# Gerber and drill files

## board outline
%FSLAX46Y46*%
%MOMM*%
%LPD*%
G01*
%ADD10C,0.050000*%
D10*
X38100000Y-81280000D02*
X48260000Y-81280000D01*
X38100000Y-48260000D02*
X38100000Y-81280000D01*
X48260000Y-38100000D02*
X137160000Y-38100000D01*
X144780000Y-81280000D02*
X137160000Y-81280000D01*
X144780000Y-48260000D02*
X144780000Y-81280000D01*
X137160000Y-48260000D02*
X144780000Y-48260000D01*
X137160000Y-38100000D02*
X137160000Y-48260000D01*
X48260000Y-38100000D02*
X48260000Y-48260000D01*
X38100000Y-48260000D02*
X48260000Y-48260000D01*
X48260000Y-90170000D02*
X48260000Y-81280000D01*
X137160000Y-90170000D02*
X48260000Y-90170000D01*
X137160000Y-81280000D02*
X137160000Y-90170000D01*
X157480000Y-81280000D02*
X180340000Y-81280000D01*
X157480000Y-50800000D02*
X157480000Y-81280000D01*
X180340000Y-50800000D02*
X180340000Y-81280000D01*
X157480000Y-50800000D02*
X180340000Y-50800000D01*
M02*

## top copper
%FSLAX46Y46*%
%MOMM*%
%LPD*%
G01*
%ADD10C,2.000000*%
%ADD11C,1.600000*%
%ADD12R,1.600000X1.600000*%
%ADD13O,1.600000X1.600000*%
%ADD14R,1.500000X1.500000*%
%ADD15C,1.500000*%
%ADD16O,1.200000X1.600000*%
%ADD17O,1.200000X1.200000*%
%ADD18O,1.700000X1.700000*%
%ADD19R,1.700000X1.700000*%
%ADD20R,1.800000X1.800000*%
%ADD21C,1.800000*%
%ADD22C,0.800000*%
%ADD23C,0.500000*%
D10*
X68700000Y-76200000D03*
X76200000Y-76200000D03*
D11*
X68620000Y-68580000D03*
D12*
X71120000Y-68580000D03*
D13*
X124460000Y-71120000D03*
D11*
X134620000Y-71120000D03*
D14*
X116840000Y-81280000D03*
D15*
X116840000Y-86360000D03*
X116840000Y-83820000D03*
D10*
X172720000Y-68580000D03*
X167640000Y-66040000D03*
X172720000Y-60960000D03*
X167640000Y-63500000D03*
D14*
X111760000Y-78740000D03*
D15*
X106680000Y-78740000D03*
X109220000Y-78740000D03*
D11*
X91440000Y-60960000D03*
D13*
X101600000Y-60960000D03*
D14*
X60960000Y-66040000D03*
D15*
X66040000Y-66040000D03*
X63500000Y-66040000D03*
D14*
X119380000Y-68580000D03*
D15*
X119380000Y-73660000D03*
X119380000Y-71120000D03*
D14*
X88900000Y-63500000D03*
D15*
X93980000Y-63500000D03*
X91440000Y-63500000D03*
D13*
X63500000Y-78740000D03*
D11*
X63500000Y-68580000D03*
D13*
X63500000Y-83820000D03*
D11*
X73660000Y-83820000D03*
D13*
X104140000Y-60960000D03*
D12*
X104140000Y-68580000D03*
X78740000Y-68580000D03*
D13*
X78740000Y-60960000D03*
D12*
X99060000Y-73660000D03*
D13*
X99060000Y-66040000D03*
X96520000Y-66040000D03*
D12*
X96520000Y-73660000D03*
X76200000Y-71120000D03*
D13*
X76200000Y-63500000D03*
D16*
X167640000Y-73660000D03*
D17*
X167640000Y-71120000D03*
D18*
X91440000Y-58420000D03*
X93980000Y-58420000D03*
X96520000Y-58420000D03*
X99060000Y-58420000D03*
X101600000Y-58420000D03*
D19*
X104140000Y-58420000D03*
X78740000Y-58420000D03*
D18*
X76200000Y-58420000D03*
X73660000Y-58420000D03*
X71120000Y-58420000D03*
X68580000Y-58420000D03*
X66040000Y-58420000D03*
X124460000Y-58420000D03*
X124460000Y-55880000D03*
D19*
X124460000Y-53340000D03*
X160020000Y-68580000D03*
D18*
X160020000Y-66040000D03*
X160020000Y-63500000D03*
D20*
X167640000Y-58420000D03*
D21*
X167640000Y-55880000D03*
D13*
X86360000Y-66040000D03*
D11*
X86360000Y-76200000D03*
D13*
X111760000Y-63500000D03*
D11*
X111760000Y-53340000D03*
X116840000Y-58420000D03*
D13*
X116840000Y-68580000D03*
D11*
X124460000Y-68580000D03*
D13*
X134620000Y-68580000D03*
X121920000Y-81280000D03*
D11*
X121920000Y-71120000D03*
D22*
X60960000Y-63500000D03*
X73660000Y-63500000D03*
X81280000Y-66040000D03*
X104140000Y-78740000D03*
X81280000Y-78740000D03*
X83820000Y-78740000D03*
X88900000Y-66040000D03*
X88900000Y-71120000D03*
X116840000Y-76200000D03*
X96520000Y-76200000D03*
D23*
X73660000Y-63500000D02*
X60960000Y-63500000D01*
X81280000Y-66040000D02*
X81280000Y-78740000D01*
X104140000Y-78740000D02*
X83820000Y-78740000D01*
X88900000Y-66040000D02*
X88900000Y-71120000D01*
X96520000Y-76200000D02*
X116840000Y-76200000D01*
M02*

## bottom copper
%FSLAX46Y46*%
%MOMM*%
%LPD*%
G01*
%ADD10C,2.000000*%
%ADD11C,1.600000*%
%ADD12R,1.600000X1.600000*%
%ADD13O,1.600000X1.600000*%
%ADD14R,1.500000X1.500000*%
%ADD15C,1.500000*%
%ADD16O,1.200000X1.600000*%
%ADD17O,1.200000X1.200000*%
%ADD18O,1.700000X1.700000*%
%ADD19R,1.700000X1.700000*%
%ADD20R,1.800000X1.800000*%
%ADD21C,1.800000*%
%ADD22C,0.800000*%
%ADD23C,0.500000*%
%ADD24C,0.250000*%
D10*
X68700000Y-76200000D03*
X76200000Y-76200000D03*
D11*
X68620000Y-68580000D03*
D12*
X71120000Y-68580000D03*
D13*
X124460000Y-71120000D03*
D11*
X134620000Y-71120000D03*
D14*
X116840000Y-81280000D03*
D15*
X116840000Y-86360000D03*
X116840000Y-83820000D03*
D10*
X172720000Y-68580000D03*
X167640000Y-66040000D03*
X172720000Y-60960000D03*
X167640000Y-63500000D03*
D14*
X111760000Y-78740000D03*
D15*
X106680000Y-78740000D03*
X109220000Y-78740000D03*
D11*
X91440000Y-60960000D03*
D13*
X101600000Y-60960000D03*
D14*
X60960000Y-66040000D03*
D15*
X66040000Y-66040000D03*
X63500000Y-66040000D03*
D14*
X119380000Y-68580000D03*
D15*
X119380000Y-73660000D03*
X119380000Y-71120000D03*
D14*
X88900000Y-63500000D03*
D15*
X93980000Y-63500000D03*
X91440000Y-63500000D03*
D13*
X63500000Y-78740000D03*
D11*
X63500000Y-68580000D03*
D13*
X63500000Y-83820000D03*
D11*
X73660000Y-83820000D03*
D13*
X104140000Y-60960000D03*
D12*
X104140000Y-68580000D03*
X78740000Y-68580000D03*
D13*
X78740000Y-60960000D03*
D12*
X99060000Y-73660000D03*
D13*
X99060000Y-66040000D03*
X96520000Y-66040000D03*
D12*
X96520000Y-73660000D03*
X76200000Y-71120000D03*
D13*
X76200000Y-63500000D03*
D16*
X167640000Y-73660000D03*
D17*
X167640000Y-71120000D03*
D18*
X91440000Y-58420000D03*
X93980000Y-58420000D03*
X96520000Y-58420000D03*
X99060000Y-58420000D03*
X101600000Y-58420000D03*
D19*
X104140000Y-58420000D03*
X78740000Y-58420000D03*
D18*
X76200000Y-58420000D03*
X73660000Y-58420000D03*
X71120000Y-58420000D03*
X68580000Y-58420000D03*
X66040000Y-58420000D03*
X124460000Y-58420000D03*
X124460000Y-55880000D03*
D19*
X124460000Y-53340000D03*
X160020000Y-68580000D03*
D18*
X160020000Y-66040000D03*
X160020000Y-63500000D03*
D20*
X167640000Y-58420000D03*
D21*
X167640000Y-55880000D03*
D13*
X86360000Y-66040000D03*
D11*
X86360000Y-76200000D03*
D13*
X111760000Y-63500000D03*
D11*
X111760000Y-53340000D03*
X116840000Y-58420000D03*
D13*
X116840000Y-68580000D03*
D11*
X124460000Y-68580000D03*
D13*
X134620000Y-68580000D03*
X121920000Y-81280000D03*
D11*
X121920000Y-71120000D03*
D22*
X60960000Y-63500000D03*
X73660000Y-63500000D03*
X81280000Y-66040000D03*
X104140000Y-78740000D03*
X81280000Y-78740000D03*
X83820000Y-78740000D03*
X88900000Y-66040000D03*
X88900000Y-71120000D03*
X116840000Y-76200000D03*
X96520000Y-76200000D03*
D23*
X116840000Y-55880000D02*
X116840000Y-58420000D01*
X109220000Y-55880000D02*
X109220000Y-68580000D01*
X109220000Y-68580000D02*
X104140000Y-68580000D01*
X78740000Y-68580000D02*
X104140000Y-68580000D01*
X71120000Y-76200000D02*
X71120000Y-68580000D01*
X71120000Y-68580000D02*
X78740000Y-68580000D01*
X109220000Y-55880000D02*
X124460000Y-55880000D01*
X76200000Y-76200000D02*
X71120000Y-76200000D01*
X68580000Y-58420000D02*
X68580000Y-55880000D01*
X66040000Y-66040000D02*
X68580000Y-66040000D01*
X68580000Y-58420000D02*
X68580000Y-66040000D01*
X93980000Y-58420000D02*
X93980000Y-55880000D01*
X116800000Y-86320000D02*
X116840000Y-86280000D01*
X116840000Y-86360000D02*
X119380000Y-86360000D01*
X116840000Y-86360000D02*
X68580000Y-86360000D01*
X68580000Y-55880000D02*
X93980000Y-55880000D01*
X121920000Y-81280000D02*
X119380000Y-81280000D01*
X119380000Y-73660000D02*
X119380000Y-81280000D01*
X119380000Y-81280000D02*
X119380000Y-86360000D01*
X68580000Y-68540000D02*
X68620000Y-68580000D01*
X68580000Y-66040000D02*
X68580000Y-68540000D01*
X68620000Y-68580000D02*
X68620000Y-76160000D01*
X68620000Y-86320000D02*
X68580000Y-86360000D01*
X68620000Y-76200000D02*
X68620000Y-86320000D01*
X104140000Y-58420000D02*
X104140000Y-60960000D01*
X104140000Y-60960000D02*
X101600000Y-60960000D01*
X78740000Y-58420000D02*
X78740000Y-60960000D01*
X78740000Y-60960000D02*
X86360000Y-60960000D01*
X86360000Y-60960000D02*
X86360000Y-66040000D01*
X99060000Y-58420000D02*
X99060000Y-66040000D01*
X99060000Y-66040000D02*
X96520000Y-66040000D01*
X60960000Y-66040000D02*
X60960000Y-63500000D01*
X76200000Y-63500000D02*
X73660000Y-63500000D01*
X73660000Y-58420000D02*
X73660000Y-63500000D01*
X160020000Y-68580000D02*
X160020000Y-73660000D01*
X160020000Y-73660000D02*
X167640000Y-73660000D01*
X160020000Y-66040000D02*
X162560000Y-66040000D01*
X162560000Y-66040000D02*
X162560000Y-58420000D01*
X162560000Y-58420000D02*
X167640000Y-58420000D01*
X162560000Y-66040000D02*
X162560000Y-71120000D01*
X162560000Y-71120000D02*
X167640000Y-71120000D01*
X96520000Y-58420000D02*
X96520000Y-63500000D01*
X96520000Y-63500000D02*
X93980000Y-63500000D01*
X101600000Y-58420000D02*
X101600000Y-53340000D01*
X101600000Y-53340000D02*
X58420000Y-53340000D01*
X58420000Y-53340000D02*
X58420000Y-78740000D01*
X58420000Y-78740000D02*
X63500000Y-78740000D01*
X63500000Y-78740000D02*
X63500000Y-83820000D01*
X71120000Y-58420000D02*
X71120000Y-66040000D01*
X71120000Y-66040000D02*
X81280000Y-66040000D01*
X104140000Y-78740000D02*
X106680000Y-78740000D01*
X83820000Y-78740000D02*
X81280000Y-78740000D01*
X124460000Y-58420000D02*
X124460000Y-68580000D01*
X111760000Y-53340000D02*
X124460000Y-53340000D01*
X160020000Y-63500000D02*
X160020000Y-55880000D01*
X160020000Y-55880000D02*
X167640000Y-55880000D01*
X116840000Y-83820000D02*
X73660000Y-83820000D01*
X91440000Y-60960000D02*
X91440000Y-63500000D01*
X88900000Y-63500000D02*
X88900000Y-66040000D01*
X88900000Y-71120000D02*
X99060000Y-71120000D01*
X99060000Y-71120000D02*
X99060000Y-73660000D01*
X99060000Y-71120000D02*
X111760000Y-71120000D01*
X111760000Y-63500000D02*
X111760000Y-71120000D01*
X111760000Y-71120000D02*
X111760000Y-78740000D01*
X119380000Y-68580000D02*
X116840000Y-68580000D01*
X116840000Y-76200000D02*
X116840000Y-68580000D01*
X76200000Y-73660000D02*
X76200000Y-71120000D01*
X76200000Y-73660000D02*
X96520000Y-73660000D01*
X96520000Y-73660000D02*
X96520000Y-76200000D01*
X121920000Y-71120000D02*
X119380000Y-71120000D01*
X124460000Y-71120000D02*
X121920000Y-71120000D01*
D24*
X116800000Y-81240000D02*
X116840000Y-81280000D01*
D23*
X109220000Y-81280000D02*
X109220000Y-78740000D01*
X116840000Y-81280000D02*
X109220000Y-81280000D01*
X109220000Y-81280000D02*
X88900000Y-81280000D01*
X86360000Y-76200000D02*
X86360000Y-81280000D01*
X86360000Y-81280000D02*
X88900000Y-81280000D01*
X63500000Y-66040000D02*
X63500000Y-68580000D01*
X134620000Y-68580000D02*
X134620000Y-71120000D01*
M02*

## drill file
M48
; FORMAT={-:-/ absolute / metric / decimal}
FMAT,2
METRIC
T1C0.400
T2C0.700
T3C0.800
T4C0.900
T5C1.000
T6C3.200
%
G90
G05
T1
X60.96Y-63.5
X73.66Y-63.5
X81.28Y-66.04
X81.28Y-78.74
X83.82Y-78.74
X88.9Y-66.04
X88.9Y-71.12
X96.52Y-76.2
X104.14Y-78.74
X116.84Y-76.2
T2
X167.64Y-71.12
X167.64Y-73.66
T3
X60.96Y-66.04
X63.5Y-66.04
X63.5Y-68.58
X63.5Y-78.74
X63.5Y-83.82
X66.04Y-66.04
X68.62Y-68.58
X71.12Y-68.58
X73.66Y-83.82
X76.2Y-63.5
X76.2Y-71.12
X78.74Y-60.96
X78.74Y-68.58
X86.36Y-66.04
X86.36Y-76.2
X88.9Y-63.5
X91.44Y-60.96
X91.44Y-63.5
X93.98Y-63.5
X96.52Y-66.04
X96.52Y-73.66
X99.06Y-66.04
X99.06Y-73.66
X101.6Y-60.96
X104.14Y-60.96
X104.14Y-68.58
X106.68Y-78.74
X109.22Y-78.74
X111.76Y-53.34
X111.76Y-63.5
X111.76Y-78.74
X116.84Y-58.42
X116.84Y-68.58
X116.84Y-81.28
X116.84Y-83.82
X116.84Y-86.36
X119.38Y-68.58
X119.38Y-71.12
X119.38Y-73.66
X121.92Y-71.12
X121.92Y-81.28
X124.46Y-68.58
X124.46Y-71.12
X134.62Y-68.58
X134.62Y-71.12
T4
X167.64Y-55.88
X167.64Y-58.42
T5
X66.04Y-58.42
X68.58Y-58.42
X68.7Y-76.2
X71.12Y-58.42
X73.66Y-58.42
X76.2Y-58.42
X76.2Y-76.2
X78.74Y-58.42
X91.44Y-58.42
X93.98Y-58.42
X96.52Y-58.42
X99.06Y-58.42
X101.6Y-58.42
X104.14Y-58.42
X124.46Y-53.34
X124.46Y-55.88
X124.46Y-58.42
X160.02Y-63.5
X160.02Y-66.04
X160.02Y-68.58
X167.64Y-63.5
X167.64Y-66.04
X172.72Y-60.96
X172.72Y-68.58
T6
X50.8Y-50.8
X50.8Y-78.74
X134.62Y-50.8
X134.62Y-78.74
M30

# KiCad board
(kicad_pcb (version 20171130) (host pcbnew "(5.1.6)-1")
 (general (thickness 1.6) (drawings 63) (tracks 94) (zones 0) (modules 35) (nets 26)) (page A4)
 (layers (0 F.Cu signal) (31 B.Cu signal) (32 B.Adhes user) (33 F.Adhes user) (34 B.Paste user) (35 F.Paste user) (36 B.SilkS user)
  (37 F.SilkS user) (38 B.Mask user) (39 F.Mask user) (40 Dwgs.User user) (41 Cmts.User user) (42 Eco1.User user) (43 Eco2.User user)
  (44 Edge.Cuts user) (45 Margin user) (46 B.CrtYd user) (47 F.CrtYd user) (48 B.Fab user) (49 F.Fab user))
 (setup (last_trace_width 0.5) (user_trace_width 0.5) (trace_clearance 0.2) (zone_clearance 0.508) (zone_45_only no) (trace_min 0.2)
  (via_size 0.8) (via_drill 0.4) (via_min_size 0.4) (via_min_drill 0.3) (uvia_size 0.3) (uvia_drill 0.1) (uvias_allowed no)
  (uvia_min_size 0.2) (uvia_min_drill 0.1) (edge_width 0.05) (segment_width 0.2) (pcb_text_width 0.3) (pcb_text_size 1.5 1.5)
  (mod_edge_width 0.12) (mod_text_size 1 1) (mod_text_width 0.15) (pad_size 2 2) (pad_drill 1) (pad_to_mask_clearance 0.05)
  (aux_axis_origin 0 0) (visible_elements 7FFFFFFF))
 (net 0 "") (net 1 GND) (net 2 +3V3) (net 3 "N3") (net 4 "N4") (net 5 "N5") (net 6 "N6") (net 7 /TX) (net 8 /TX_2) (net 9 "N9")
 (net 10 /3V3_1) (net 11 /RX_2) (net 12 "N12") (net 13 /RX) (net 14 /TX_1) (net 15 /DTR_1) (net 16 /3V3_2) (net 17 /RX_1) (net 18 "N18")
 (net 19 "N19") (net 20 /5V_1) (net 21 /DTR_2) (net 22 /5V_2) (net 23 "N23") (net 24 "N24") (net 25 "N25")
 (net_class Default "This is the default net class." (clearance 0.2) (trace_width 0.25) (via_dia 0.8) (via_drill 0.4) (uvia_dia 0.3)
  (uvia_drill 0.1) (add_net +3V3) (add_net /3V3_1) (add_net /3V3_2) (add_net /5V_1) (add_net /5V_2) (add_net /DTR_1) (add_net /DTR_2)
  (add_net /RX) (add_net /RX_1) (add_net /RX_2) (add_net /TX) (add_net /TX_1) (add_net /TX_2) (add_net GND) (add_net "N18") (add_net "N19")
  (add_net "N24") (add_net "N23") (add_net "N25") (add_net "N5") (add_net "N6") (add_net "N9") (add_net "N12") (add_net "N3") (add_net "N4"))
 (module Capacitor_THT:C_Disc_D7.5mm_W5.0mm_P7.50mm (layer F.Cu) (at 76.2 76.2 180)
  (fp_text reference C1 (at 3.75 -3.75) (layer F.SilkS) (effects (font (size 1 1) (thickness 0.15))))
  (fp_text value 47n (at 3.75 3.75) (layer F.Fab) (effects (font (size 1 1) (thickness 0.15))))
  (pad 2 thru_hole circle (at 7.5 0 180) (size 2 2) (drill 1) (layers *.Cu *.Mask) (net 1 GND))
  (pad 1 thru_hole circle (at 0 0 180) (size 2 2) (drill 1) (layers *.Cu *.Mask) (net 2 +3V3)))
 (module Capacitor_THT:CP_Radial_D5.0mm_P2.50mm (layer F.Cu) (at 71.12 68.58 180)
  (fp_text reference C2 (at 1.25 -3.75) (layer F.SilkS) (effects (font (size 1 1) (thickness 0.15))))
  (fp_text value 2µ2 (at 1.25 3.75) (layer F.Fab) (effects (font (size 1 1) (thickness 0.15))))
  (pad 2 thru_hole circle (at 2.5 0 180) (size 1.6 1.6) (drill 0.8) (layers *.Cu *.Mask) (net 1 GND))
  (pad 1 thru_hole rect (at 0 0 180) (size 1.6 1.6) (drill 0.8) (layers *.Cu *.Mask) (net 2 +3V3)))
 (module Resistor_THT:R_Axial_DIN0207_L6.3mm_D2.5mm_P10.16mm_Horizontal (layer F.Cu) (at 134.62 71.12 180)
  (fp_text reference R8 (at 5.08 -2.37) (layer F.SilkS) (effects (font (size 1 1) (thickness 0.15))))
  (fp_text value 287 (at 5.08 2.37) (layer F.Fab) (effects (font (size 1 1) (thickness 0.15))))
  (pad 2 thru_hole oval (at 10.16 0 180) (size 1.6 1.6) (drill 0.8) (layers *.Cu *.Mask) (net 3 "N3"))
  (pad 1 thru_hole circle (at 0 0 180) (size 1.6 1.6) (drill 0.8) (layers *.Cu *.Mask) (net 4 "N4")))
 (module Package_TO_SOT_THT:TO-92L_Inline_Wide (layer F.Cu) (at 116.84 81.28 270)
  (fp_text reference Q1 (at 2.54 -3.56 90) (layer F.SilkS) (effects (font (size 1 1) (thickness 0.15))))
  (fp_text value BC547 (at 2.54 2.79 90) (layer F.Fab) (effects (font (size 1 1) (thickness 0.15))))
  (pad 1 thru_hole rect (at 0 0) (size 1.5 1.5) (drill 0.8) (layers *.Cu *.Mask) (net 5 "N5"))
  (pad 3 thru_hole circle (at 5.08 0) (size 1.5 1.5) (drill 0.8) (layers *.Cu *.Mask) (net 1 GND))
  (pad 2 thru_hole circle (at 2.54 0) (size 1.5 1.5) (drill 0.8) (layers *.Cu *.Mask) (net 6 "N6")))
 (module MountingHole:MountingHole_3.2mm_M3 (layer F.Cu) (at 50.8 50.8)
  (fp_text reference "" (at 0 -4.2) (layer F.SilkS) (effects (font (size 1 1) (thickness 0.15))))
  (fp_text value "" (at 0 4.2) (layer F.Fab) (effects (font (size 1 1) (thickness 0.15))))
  (pad 1 np_thru_hole circle (at 0 0) (size 3.2 3.2) (drill 3.2) (layers *.Cu *.Mask)))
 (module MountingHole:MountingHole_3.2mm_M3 (layer F.Cu) (at 134.62 78.74)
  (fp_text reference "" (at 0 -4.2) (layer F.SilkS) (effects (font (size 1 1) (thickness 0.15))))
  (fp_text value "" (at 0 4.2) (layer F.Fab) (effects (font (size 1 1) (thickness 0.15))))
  (pad 1 np_thru_hole circle (at 0 0) (size 3.2 3.2) (drill 3.2) (layers *.Cu *.Mask)))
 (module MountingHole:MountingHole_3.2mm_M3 (layer F.Cu) (at 134.62 50.8)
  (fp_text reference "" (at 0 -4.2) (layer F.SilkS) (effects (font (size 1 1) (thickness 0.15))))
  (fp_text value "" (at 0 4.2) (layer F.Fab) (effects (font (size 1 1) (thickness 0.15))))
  (pad 1 np_thru_hole circle (at 0 0) (size 3.2 3.2) (drill 3.2) (layers *.Cu *.Mask)))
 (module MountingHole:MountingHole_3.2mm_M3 (layer F.Cu) (at 50.8 78.74)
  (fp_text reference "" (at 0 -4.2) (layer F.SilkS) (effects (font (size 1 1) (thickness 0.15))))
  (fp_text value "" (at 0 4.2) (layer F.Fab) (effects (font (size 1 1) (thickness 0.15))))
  (pad 1 np_thru_hole circle (at 0 0) (size 3.2 3.2) (drill 3.2) (layers *.Cu *.Mask)))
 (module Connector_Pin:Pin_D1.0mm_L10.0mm (layer F.Cu) (at 172.72 68.58)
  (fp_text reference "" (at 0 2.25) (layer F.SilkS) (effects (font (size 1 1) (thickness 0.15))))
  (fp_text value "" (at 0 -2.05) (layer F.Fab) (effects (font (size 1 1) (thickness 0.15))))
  (pad V thru_hole circle (at 0 0) (size 2 2) (drill 1) (layers *.Cu *.Mask)))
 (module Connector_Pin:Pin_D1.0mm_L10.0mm (layer F.Cu) (at 167.64 66.04)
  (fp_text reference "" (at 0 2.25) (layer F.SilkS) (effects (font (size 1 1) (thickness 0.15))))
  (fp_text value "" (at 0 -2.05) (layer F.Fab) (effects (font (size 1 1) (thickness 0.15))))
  (pad V thru_hole circle (at 0 0) (size 2 2) (drill 1) (layers *.Cu *.Mask)))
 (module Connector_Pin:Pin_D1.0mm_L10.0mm (layer F.Cu) (at 172.72 60.96)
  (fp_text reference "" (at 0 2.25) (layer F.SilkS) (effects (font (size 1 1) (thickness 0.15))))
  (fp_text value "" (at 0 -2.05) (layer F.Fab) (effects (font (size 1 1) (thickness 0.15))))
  (pad V thru_hole circle (at 0 0) (size 2 2) (drill 1) (layers *.Cu *.Mask)))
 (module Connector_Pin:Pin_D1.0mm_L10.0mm (layer F.Cu) (at 167.64 63.5)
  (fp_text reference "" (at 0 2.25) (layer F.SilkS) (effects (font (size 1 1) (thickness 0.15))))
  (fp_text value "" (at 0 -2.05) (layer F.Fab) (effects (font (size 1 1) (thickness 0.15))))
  (pad V thru_hole circle (at 0 0) (size 2 2) (drill 1) (layers *.Cu *.Mask)))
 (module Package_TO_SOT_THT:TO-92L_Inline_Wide (layer F.Cu) (at 111.76 78.74 180)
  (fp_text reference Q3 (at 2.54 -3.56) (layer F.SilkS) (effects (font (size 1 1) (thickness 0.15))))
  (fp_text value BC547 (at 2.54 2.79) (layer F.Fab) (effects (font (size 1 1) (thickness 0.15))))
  (pad 1 thru_hole rect (at 0 0 270) (size 1.5 1.5) (drill 0.8) (layers *.Cu *.Mask) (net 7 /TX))
  (pad 3 thru_hole circle (at 5.08 0 270) (size 1.5 1.5) (drill 0.8) (layers *.Cu *.Mask) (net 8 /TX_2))
  (pad 2 thru_hole circle (at 2.54 0 270) (size 1.5 1.5) (drill 0.8) (layers *.Cu *.Mask) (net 5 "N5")))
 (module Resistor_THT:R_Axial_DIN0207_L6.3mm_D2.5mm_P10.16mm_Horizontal (layer F.Cu) (at 91.44 60.96)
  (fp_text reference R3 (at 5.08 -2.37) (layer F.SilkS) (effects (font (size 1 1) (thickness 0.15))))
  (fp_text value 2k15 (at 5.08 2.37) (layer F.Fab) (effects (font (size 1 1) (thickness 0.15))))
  (pad 1 thru_hole circle (at 0 0) (size 1.6 1.6) (drill 0.8) (layers *.Cu *.Mask) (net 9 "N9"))
  (pad 2 thru_hole oval (at 10.16 0) (size 1.6 1.6) (drill 0.8) (layers *.Cu *.Mask) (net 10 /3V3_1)))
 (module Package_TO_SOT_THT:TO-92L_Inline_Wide (layer F.Cu) (at 60.96 66.04)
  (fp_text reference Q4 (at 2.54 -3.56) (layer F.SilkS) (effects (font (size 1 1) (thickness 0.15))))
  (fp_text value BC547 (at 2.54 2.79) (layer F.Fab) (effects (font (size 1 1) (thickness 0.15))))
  (pad 1 thru_hole rect (at 0 0 90) (size 1.5 1.5) (drill 0.8) (layers *.Cu *.Mask) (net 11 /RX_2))
  (pad 3 thru_hole circle (at 5.08 0 90) (size 1.5 1.5) (drill 0.8) (layers *.Cu *.Mask) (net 1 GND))
  (pad 2 thru_hole circle (at 2.54 0 90) (size 1.5 1.5) (drill 0.8) (layers *.Cu *.Mask) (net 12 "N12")))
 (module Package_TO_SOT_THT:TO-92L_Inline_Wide (layer F.Cu) (at 119.38 68.58 270)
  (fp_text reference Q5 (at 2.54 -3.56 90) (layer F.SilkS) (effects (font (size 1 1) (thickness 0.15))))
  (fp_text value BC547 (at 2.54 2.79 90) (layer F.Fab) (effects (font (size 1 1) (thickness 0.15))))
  (pad 1 thru_hole rect (at 0 0) (size 1.5 1.5) (drill 0.8) (layers *.Cu *.Mask) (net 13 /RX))
  (pad 3 thru_hole circle (at 5.08 0) (size 1.5 1.5) (drill 0.8) (layers *.Cu *.Mask) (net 1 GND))
  (pad 2 thru_hole circle (at 2.54 0) (size 1.5 1.5) (drill 0.8) (layers *.Cu *.Mask) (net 3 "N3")))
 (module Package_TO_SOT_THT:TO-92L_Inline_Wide (layer F.Cu) (at 88.9 63.5)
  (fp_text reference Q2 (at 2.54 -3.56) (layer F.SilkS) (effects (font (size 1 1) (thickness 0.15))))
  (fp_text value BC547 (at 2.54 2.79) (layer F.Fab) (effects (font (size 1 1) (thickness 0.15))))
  (pad 1 thru_hole rect (at 0 0 90) (size 1.5 1.5) (drill 0.8) (layers *.Cu *.Mask) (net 7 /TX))
  (pad 3 thru_hole circle (at 5.08 0 90) (size 1.5 1.5) (drill 0.8) (layers *.Cu *.Mask) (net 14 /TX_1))
  (pad 2 thru_hole circle (at 2.54 0 90) (size 1.5 1.5) (drill 0.8) (layers *.Cu *.Mask) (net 9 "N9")))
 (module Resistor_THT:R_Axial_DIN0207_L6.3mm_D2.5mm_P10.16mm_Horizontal (layer F.Cu) (at 63.5 68.58 270)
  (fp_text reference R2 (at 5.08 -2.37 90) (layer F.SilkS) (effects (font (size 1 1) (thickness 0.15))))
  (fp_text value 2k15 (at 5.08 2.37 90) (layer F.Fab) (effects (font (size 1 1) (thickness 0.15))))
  (pad 2 thru_hole oval (at 10.16 0 270) (size 1.6 1.6) (drill 0.8) (layers *.Cu *.Mask) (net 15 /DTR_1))
  (pad 1 thru_hole circle (at 0 0 270) (size 1.6 1.6) (drill 0.8) (layers *.Cu *.Mask) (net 12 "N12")))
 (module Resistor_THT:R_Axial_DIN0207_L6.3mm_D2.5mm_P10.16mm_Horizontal (layer F.Cu) (at 73.66 83.82 180)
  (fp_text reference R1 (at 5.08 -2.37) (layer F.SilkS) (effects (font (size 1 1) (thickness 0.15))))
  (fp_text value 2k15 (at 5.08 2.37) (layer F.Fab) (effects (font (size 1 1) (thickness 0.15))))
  (pad 2 thru_hole oval (at 10.16 0 180) (size 1.6 1.6) (drill 0.8) (layers *.Cu *.Mask) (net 15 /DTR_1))
  (pad 1 thru_hole circle (at 0 0 180) (size 1.6 1.6) (drill 0.8) (layers *.Cu *.Mask) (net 6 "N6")))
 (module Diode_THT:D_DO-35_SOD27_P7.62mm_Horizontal (layer F.Cu) (at 104.14 68.58 90)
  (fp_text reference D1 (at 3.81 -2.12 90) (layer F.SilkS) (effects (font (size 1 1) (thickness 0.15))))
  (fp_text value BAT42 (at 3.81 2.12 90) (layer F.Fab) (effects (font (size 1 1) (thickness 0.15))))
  (pad 2 thru_hole oval (at 7.62 0 90) (size 1.6 1.6) (drill 0.8) (layers *.Cu *.Mask) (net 10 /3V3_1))
  (pad 1 thru_hole rect (at 0 0 90) (size 1.6 1.6) (drill 0.8) (layers *.Cu *.Mask) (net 2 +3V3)))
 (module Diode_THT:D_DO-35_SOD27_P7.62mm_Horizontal (layer F.Cu) (at 78.74 68.58 90)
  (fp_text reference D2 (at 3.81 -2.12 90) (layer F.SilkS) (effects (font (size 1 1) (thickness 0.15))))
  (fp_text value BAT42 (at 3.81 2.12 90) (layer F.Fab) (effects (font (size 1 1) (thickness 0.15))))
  (pad 1 thru_hole rect (at 0 0 90) (size 1.6 1.6) (drill 0.8) (layers *.Cu *.Mask) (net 2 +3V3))
  (pad 2 thru_hole oval (at 7.62 0 90) (size 1.6 1.6) (drill 0.8) (layers *.Cu *.Mask) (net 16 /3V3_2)))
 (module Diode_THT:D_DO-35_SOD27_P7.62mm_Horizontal (layer F.Cu) (at 99.06 73.66 90)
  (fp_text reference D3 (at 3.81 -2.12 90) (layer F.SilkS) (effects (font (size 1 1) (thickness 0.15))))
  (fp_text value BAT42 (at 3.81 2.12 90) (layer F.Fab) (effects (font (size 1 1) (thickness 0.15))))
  (pad 1 thru_hole rect (at 0 0 90) (size 1.6 1.6) (drill 0.8) (layers *.Cu *.Mask) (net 7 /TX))
  (pad 2 thru_hole oval (at 7.62 0 90) (size 1.6 1.6) (drill 0.8) (layers *.Cu *.Mask) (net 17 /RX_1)))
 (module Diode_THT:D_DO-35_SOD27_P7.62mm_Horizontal (layer F.Cu) (at 96.52 73.66 90)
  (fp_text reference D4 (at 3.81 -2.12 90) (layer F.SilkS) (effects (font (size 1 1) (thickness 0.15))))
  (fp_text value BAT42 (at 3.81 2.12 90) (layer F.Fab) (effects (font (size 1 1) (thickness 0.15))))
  (pad 2 thru_hole oval (at 7.62 0 90) (size 1.6 1.6) (drill 0.8) (layers *.Cu *.Mask) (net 17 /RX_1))
  (pad 1 thru_hole rect (at 0 0 90) (size 1.6 1.6) (drill 0.8) (layers *.Cu *.Mask) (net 13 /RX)))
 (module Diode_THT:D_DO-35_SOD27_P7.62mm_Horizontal (layer F.Cu) (at 76.2 71.12 90)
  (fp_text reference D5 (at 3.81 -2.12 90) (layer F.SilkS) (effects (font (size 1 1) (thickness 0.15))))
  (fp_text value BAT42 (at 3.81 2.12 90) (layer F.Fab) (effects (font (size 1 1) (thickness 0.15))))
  (pad 1 thru_hole rect (at 0 0 90) (size 1.6 1.6) (drill 0.8) (layers *.Cu *.Mask) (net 13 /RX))
  (pad 2 thru_hole oval (at 7.62 0 90) (size 1.6 1.6) (drill 0.8) (layers *.Cu *.Mask) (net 11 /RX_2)))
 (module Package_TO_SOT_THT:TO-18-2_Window (layer F.Cu) (at 167.64 73.66 90)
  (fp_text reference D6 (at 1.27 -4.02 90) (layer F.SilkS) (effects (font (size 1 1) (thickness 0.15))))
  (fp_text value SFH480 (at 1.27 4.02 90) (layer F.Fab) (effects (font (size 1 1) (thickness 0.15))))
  (pad 1 thru_hole oval (at 0 0 90) (size 1.6 1.2) (drill 0.7) (layers *.Cu *.Mask) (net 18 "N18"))
  (pad 2 thru_hole oval (at 2.54 0 90) (size 1.2 1.2) (drill 0.7) (layers *.Cu *.Mask) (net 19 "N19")))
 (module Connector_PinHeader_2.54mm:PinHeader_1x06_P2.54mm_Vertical (layer F.Cu) (at 104.14 58.42 270)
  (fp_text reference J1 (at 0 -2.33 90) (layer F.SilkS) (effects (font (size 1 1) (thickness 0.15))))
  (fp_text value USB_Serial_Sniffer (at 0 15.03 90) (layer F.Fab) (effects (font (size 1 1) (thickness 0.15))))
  (pad 6 thru_hole oval (at 0 12.7 270) (size 1.7 1.7) (drill 1) (layers *.Cu *.Mask) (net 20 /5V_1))
  (pad 5 thru_hole oval (at 0 10.16 270) (size 1.7 1.7) (drill 1) (layers *.Cu *.Mask) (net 1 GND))
  (pad 4 thru_hole oval (at 0 7.62 270) (size 1.7 1.7) (drill 1) (layers *.Cu *.Mask) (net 14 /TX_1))
  (pad 3 thru_hole oval (at 0 5.08 270) (size 1.7 1.7) (drill 1) (layers *.Cu *.Mask) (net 17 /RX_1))
  (pad 2 thru_hole oval (at 0 2.54 270) (size 1.7 1.7) (drill 1) (layers *.Cu *.Mask) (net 15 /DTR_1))
  (pad 1 thru_hole rect (at 0 0 270) (size 1.7 1.7) (drill 1) (layers *.Cu *.Mask) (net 10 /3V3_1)))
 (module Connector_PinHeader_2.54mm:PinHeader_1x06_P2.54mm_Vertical (layer F.Cu) (at 78.74 58.42 270)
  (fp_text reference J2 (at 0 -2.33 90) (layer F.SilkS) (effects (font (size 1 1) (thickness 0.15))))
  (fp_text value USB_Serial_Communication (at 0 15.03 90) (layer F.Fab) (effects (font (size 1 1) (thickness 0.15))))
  (pad 1 thru_hole rect (at 0 0 270) (size 1.7 1.7) (drill 1) (layers *.Cu *.Mask) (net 16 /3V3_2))
  (pad 2 thru_hole oval (at 0 2.54 270) (size 1.7 1.7) (drill 1) (layers *.Cu *.Mask) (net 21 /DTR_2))
  (pad 3 thru_hole oval (at 0 5.08 270) (size 1.7 1.7) (drill 1) (layers *.Cu *.Mask) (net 11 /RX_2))
  (pad 4 thru_hole oval (at 0 7.62 270) (size 1.7 1.7) (drill 1) (layers *.Cu *.Mask) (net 8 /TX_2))
  (pad 5 thru_hole oval (at 0 10.16 270) (size 1.7 1.7) (drill 1) (layers *.Cu *.Mask) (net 1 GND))
  (pad 6 thru_hole oval (at 0 12.7 270) (size 1.7 1.7) (drill 1) (layers *.Cu *.Mask) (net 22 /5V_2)))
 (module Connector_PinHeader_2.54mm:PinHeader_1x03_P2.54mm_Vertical (layer F.Cu) (at 124.46 53.34)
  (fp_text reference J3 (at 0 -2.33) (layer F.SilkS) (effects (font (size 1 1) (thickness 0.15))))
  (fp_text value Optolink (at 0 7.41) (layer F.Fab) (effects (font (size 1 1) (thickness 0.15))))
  (pad 3 thru_hole oval (at 0 5.08) (size 1.7 1.7) (drill 1) (layers *.Cu *.Mask) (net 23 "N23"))
  (pad 2 thru_hole oval (at 0 2.54) (size 1.7 1.7) (drill 1) (layers *.Cu *.Mask) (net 2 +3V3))
  (pad 1 thru_hole rect (at 0 0) (size 1.7 1.7) (drill 1) (layers *.Cu *.Mask) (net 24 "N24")))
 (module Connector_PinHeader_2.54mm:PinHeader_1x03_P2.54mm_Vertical (layer F.Cu) (at 160.02 68.58 180)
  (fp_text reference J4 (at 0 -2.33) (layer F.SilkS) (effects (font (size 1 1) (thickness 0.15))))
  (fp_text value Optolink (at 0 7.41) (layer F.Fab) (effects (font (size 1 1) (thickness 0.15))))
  (pad 1 thru_hole rect (at 0 0 180) (size 1.7 1.7) (drill 1) (layers *.Cu *.Mask) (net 18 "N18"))
  (pad 2 thru_hole oval (at 0 2.54 180) (size 1.7 1.7) (drill 1) (layers *.Cu *.Mask) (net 19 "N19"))
  (pad 3 thru_hole oval (at 0 5.08 180) (size 1.7 1.7) (drill 1) (layers *.Cu *.Mask) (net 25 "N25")))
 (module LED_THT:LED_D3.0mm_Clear (layer F.Cu) (at 167.64 58.42 90)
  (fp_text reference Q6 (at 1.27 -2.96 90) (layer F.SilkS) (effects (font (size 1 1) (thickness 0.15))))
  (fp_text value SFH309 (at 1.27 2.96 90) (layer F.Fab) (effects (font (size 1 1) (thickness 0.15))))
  (pad 1 thru_hole rect (at 0 0 90) (size 1.8 1.8) (drill 0.9) (layers *.Cu *.Mask) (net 19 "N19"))
  (pad 2 thru_hole circle (at 2.54 0 90) (size 1.8 1.8) (drill 0.9) (layers *.Cu *.Mask) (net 25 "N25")))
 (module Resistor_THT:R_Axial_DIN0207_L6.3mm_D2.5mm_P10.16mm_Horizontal (layer F.Cu) (at 86.36 76.2 90)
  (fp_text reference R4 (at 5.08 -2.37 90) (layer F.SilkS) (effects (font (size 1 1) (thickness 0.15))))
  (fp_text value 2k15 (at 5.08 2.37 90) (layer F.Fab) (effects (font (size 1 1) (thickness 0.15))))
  (pad 2 thru_hole oval (at 10.16 0 90) (size 1.6 1.6) (drill 0.8) (layers *.Cu *.Mask) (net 16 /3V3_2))
  (pad 1 thru_hole circle (at 0 0 90) (size 1.6 1.6) (drill 0.8) (layers *.Cu *.Mask) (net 5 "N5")))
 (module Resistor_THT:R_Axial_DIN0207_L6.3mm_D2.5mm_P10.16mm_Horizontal (layer F.Cu) (at 111.76 53.34 270)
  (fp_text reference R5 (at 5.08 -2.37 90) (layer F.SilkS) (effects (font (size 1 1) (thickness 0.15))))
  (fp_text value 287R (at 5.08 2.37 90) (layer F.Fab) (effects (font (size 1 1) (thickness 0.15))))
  (pad 2 thru_hole oval (at 10.16 0 270) (size 1.6 1.6) (drill 0.8) (layers *.Cu *.Mask) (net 7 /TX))
  (pad 1 thru_hole circle (at 0 0 270) (size 1.6 1.6) (drill 0.8) (layers *.Cu *.Mask) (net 24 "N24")))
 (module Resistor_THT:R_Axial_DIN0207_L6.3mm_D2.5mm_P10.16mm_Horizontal (layer F.Cu) (at 116.84 58.42 270)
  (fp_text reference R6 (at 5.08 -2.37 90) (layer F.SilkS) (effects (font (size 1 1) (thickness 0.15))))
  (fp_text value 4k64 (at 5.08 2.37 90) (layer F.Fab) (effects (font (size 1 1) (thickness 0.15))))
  (pad 1 thru_hole circle (at 0 0 270) (size 1.6 1.6) (drill 0.8) (layers *.Cu *.Mask) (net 2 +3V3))
  (pad 2 thru_hole oval (at 10.16 0 270) (size 1.6 1.6) (drill 0.8) (layers *.Cu *.Mask) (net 13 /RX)))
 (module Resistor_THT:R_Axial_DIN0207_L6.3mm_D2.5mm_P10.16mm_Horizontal (layer F.Cu) (at 124.46 68.58)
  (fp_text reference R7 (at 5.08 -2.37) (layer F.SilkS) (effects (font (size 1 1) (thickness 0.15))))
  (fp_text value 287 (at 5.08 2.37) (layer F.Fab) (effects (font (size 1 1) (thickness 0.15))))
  (pad 1 thru_hole circle (at 0 0) (size 1.6 1.6) (drill 0.8) (layers *.Cu *.Mask) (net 23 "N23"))
  (pad 2 thru_hole oval (at 10.16 0) (size 1.6 1.6) (drill 0.8) (layers *.Cu *.Mask) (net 4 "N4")))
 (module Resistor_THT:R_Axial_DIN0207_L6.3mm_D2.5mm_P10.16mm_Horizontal (layer F.Cu) (at 121.92 71.12 270)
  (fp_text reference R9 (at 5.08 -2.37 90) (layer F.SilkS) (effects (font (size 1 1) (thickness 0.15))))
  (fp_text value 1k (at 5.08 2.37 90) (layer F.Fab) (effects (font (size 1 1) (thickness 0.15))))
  (pad 2 thru_hole oval (at 10.16 0 270) (size 1.6 1.6) (drill 0.8) (layers *.Cu *.Mask) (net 1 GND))
  (pad 1 thru_hole circle (at 0 0 270) (size 1.6 1.6) (drill 0.8) (layers *.Cu *.Mask) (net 3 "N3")))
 (gr_line (start 38.1 81.28) (end 48.26 81.28) (layer Edge.Cuts) (width 0.05))
 (gr_line (start 38.1 48.26) (end 38.1 81.28) (layer Edge.Cuts) (width 0.05))
 (gr_line (start 48.26 38.1) (end 137.16 38.1) (layer Edge.Cuts) (width 0.05))
 (gr_line (start 144.78 81.28) (end 137.16 81.28) (layer Edge.Cuts) (width 0.05))
 (gr_line (start 144.78 48.26) (end 144.78 81.28) (layer Edge.Cuts) (width 0.05))
 (gr_line (start 137.16 48.26) (end 144.78 48.26) (layer Edge.Cuts) (width 0.05))
 (gr_line (start 137.16 38.1) (end 137.16 48.26) (layer Edge.Cuts) (width 0.05))
 (gr_line (start 48.26 38.1) (end 48.26 48.26) (layer Edge.Cuts) (width 0.05))
 (gr_line (start 38.1 48.26) (end 48.26 48.26) (layer Edge.Cuts) (width 0.05))
 (gr_line (start 48.26 90.17) (end 48.26 81.28) (layer Edge.Cuts) (width 0.05))
 (gr_line (start 137.16 90.17) (end 48.26 90.17) (layer Edge.Cuts) (width 0.05))
 (gr_line (start 137.16 81.28) (end 137.16 90.17) (layer Edge.Cuts) (width 0.05))
 (gr_line (start 157.48 81.28) (end 180.34 81.28) (layer Edge.Cuts) (width 0.05))
 (gr_line (start 157.48 50.8) (end 157.48 81.28) (layer Edge.Cuts) (width 0.05))
 (gr_line (start 180.34 50.8) (end 180.34 81.28) (layer Edge.Cuts) (width 0.05))
 (gr_line (start 157.48 50.8) (end 180.34 50.8) (layer Edge.Cuts) (width 0.05))
 (segment (start 116.84 55.88) (end 116.84 58.42) (width 0.5) (layer B.Cu) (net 2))
 (segment (start 109.22 55.88) (end 109.22 68.58) (width 0.5) (layer B.Cu) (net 2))
 (segment (start 109.22 68.58) (end 104.14 68.58) (width 0.5) (layer B.Cu) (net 2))
 (segment (start 78.74 68.58) (end 104.14 68.58) (width 0.5) (layer B.Cu) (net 2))
 (segment (start 71.12 76.2) (end 71.12 68.58) (width 0.5) (layer B.Cu) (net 2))
 (segment (start 71.12 68.58) (end 78.74 68.58) (width 0.5) (layer B.Cu) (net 2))
 (segment (start 109.22 55.88) (end 124.46 55.88) (width 0.5) (layer B.Cu) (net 2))
 (segment (start 76.2 76.2) (end 71.12 76.2) (width 0.5) (layer B.Cu) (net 2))
 (segment (start 68.58 58.42) (end 68.58 55.88) (width 0.5) (layer B.Cu) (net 1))
 (segment (start 66.04 66.04) (end 68.58 66.04) (width 0.5) (layer B.Cu) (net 1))
 (segment (start 68.58 58.42) (end 68.58 66.04) (width 0.5) (layer B.Cu) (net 1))
 (segment (start 93.98 58.42) (end 93.98 55.88) (width 0.5) (layer B.Cu) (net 1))
 (segment (start 116.8 86.32) (end 116.84 86.28) (width 0.5) (layer B.Cu) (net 1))
 (segment (start 116.84 86.36) (end 119.38 86.36) (width 0.5) (layer B.Cu) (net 1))
 (segment (start 116.84 86.36) (end 68.58 86.36) (width 0.5) (layer B.Cu) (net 1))
 (segment (start 68.58 55.88) (end 93.98 55.88) (width 0.5) (layer B.Cu) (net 1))
 (segment (start 121.92 81.28) (end 119.38 81.28) (width 0.5) (layer B.Cu) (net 1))
 (segment (start 119.38 73.66) (end 119.38 81.28) (width 0.5) (layer B.Cu) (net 1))
 (segment (start 119.38 81.28) (end 119.38 86.36) (width 0.5) (layer B.Cu) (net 1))
 (segment (start 68.58 68.54) (end 68.62 68.58) (width 0.5) (layer B.Cu) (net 1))
 (segment (start 68.58 66.04) (end 68.58 68.54) (width 0.5) (layer B.Cu) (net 1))
 (segment (start 68.62 68.58) (end 68.62 76.16) (width 0.5) (layer B.Cu) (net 1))
 (segment (start 68.62 86.32) (end 68.58 86.36) (width 0.5) (layer B.Cu) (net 1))
 (segment (start 68.62 76.2) (end 68.62 86.32) (width 0.5) (layer B.Cu) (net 1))
 (segment (start 104.14 58.42) (end 104.14 60.96) (width 0.5) (layer B.Cu) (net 10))
 (segment (start 104.14 60.96) (end 101.6 60.96) (width 0.5) (layer B.Cu) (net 10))
 (segment (start 78.74 58.42) (end 78.74 60.96) (width 0.5) (layer B.Cu) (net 16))
 (segment (start 78.74 60.96) (end 86.36 60.96) (width 0.5) (layer B.Cu) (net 16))
 (segment (start 86.36 60.96) (end 86.36 66.04) (width 0.5) (layer B.Cu) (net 16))
 (segment (start 99.06 58.42) (end 99.06 66.04) (width 0.5) (layer B.Cu) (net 17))
 (segment (start 99.06 66.04) (end 96.52 66.04) (width 0.5) (layer B.Cu) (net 17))
 (via (at 60.96 63.5) (size 0.8) (drill 0.4) (layers F.Cu B.Cu) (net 11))
 (segment (start 60.96 66.04) (end 60.96 63.5) (width 0.5) (layer B.Cu) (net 11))
 (via (at 73.66 63.5) (size 0.8) (drill 0.4) (layers F.Cu B.Cu) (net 11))
 (segment (start 76.2 63.5) (end 73.66 63.5) (width 0.5) (layer B.Cu) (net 11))
 (segment (start 73.66 63.5) (end 60.96 63.5) (width 0.5) (layer F.Cu) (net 11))
 (segment (start 73.66 58.42) (end 73.66 63.5) (width 0.5) (layer B.Cu) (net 11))
 (segment (start 160.02 68.58) (end 160.02 73.66) (width 0.5) (layer B.Cu) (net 18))
 (segment (start 160.02 73.66) (end 167.64 73.66) (width 0.5) (layer B.Cu) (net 18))
 (segment (start 160.02 66.04) (end 162.56 66.04) (width 0.5) (layer B.Cu) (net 19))
 (segment (start 162.56 66.04) (end 162.56 58.42) (width 0.5) (layer B.Cu) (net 19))
 (segment (start 162.56 58.42) (end 167.64 58.42) (width 0.5) (layer B.Cu) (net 19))
 (segment (start 162.56 66.04) (end 162.56 71.12) (width 0.5) (layer B.Cu) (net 19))
 (segment (start 162.56 71.12) (end 167.64 71.12) (width 0.5) (layer B.Cu) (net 19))
 (segment (start 96.52 58.42) (end 96.52 63.5) (width 0.5) (layer B.Cu) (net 14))
 (segment (start 96.52 63.5) (end 93.98 63.5) (width 0.5) (layer B.Cu) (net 14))
 (segment (start 101.6 58.42) (end 101.6 53.34) (width 0.5) (layer B.Cu) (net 15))
 (segment (start 101.6 53.34) (end 58.42 53.34) (width 0.5) (layer B.Cu) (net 15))
 (segment (start 58.42 53.34) (end 58.42 78.74) (width 0.5) (layer B.Cu) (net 15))
 (segment (start 58.42 78.74) (end 63.5 78.74) (width 0.5) (layer B.Cu) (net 15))
 (segment (start 63.5 78.74) (end 63.5 83.82) (width 0.5) (layer B.Cu) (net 15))
 (segment (start 71.12 58.42) (end 71.12 66.04) (width 0.5) (layer B.Cu) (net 8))
 (via (at 81.28 66.04) (size 0.8) (drill 0.4) (layers F.Cu B.Cu) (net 8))
 (segment (start 71.12 66.04) (end 81.28 66.04) (width 0.5) (layer B.Cu) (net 8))
 (via (at 104.14 78.74) (size 0.8) (drill 0.4) (layers F.Cu B.Cu) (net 8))
 (segment (start 104.14 78.74) (end 106.68 78.74) (width 0.5) (layer B.Cu) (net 8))
 (via (at 81.28 78.74) (size 0.8) (drill 0.4) (layers F.Cu B.Cu) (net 8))
 (segment (start 81.28 66.04) (end 81.28 78.74) (width 0.5) (layer F.Cu) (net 8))
 (via (at 83.82 78.74) (size 0.8) (drill 0.4) (layers F.Cu B.Cu) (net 8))
 (segment (start 104.14 78.74) (end 83.82 78.74) (width 0.5) (layer F.Cu) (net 8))
 (segment (start 83.82 78.74) (end 81.28 78.74) (width 0.5) (layer B.Cu) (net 8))
 (segment (start 124.46 58.42) (end 124.46 68.58) (width 0.5) (layer B.Cu) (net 23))
 (segment (start 111.76 53.34) (end 124.46 53.34) (width 0.5) (layer B.Cu) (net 24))
 (segment (start 160.02 63.5) (end 160.02 55.88) (width 0.5) (layer B.Cu) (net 25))
 (segment (start 160.02 55.88) (end 167.64 55.88) (width 0.5) (layer B.Cu) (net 25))
 (segment (start 116.84 83.82) (end 73.66 83.82) (width 0.5) (layer B.Cu) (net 6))
 (segment (start 91.44 60.96) (end 91.44 63.5) (width 0.5) (layer B.Cu) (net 9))
 (via (at 88.9 66.04) (size 0.8) (drill 0.4) (layers F.Cu B.Cu) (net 7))
 (segment (start 88.9 63.5) (end 88.9 66.04) (width 0.5) (layer B.Cu) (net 7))
 (via (at 88.9 71.12) (size 0.8) (drill 0.4) (layers F.Cu B.Cu) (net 7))
 (segment (start 88.9 66.04) (end 88.9 71.12) (width 0.5) (layer F.Cu) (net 7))
 (segment (start 88.9 71.12) (end 99.06 71.12) (width 0.5) (layer B.Cu) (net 7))
 (segment (start 99.06 71.12) (end 99.06 73.66) (width 0.5) (layer B.Cu) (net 7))
 (segment (start 99.06 71.12) (end 111.76 71.12) (width 0.5) (layer B.Cu) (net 7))
 (segment (start 111.76 63.5) (end 111.76 71.12) (width 0.5) (layer B.Cu) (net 7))
 (segment (start 111.76 71.12) (end 111.76 78.74) (width 0.5) (layer B.Cu) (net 7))
 (segment (start 119.38 68.58) (end 116.84 68.58) (width 0.5) (layer B.Cu) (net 13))
 (via (at 116.84 76.2) (size 0.8) (drill 0.4) (layers F.Cu B.Cu) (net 13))
 (segment (start 116.84 76.2) (end 116.84 68.58) (width 0.5) (layer B.Cu) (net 13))
 (segment (start 76.2 73.66) (end 76.2 71.12) (width 0.5) (layer B.Cu) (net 13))
 (segment (start 76.2 73.66) (end 96.52 73.66) (width 0.5) (layer B.Cu) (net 13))
 (via (at 96.52 76.2) (size 0.8) (drill 0.4) (layers F.Cu B.Cu) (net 13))
 (segment (start 96.52 73.66) (end 96.52 76.2) (width 0.5) (layer B.Cu) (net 13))
 (segment (start 96.52 76.2) (end 116.84 76.2) (width 0.5) (layer F.Cu) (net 13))
 (segment (start 121.92 71.12) (end 119.38 71.12) (width 0.5) (layer B.Cu) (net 3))
 (segment (start 124.46 71.12) (end 121.92 71.12) (width 0.5) (layer B.Cu) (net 3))
 (segment (start 116.8 81.24) (end 116.84 81.28) (width 0.25) (layer B.Cu) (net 5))
 (segment (start 109.22 81.28) (end 109.22 78.74) (width 0.5) (layer B.Cu) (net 5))
 (segment (start 116.84 81.28) (end 109.22 81.28) (width 0.5) (layer B.Cu) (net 5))
 (segment (start 109.22 81.28) (end 88.9 81.28) (width 0.5) (layer B.Cu) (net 5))
 (segment (start 86.36 76.2) (end 86.36 81.28) (width 0.5) (layer B.Cu) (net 5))
 (segment (start 86.36 81.28) (end 88.9 81.28) (width 0.5) (layer B.Cu) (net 5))
 (segment (start 63.5 66.04) (end 63.5 68.58) (width 0.5) (layer B.Cu) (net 12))
 (segment (start 134.62 68.58) (end 134.62 71.12) (width 0.5) (layer B.Cu) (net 4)))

